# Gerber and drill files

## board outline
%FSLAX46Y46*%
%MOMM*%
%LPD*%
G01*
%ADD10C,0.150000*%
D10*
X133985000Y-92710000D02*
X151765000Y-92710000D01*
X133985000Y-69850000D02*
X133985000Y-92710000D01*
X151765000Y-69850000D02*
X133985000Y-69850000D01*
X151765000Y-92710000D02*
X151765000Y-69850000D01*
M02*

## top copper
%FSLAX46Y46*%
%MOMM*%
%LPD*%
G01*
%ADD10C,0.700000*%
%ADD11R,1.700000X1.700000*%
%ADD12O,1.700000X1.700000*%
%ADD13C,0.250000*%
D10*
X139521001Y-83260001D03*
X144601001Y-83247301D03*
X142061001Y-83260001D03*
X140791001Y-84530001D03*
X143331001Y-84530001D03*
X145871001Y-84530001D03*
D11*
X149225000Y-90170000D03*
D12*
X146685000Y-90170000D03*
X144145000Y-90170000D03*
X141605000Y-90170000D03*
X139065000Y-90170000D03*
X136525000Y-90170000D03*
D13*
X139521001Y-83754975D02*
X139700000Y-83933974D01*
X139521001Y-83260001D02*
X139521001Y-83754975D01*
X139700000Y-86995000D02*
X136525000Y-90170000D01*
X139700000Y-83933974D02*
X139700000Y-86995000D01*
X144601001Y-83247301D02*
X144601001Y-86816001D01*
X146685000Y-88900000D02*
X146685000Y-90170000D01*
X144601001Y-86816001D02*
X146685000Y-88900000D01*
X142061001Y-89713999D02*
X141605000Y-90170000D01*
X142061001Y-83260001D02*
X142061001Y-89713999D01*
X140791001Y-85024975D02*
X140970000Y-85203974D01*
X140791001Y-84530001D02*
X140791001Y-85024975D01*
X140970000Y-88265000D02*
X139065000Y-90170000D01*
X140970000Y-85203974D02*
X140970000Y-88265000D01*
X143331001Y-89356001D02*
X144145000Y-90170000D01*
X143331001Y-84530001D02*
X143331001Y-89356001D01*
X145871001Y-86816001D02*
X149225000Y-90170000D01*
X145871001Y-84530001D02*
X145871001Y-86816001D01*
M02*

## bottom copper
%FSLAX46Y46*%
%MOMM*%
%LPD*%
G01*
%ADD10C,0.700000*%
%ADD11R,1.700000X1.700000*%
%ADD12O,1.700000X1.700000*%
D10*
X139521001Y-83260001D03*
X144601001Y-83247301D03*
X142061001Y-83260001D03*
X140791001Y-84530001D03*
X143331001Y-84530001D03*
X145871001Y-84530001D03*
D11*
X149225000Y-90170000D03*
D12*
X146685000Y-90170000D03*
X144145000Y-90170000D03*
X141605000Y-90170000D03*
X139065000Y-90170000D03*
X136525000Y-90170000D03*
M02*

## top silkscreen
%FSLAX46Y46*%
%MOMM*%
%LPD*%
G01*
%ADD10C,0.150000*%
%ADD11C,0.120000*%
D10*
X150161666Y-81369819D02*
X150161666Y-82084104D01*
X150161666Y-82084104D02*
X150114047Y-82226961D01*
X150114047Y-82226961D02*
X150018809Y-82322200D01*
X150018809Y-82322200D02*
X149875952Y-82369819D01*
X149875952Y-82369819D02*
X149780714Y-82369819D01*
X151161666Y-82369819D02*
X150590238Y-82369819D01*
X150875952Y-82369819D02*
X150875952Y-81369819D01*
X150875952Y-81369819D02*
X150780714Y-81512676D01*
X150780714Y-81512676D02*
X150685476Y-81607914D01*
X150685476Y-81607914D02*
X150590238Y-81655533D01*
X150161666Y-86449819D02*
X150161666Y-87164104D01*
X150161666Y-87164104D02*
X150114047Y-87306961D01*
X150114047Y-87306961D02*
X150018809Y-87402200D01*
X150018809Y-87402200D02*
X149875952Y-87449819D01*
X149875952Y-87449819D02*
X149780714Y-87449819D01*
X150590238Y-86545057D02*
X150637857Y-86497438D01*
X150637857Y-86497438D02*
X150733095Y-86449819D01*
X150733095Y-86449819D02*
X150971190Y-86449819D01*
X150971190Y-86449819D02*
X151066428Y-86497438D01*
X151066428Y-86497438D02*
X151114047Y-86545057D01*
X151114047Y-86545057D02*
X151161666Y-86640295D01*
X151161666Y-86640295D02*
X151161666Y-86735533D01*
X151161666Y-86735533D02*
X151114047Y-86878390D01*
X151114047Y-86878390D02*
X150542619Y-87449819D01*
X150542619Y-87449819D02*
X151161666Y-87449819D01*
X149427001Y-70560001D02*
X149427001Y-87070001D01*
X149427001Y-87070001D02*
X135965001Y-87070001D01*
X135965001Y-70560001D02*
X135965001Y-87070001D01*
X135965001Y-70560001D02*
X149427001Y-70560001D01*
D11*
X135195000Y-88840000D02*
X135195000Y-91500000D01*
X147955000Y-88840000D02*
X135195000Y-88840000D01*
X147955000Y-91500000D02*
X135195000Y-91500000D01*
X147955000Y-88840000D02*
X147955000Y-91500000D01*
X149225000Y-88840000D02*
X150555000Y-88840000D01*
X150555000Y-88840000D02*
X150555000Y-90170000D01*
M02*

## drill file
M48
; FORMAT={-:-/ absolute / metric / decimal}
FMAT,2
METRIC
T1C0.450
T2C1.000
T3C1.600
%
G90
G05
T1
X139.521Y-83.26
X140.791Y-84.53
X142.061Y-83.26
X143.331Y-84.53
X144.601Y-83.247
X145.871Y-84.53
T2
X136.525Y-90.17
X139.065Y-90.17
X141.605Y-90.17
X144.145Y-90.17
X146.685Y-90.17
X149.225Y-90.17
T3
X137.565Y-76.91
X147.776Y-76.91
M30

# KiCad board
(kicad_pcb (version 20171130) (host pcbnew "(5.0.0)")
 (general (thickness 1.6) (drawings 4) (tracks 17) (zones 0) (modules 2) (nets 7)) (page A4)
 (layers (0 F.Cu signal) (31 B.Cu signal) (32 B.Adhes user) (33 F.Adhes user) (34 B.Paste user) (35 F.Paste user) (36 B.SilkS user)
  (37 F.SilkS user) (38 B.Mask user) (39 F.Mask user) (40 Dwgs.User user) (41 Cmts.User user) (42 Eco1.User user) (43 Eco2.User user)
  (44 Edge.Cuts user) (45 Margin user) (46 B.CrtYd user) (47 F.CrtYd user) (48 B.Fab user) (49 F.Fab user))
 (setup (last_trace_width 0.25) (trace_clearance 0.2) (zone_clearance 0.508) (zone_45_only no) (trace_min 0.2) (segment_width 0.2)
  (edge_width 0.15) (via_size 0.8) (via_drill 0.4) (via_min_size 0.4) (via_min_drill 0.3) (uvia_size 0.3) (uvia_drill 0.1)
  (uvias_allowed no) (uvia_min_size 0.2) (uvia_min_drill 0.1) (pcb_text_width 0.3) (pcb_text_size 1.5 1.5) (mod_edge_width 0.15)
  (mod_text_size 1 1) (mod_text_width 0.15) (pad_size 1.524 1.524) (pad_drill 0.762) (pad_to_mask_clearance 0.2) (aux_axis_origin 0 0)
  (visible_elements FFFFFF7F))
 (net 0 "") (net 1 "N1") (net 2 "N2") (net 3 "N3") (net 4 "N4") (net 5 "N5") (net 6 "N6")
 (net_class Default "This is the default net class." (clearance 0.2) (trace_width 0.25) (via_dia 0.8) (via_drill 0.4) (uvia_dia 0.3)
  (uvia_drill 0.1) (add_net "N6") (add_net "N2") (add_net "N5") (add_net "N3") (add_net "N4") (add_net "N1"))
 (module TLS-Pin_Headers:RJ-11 (layer F.Cu) (at 142.696001 83.260001)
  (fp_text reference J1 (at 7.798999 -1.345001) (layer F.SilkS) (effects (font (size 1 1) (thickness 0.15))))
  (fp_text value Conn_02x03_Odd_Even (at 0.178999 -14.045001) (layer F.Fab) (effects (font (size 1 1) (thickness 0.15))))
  (fp_line (start 6.731 -12.7) (end 6.731 3.81) (layer F.SilkS) (width 0.15))
  (fp_line (start 6.731 3.81) (end -6.731 3.81) (layer F.SilkS) (width 0.15))
  (fp_line (start -6.731 -12.7) (end -6.731 3.81) (layer F.SilkS) (width 0.15))
  (fp_line (start -6.731 -12.7) (end 6.731 -12.7) (layer F.SilkS) (width 0.15))
  (pad "" np_thru_hole circle (at 5.08 -6.35) (size 1.6 1.6) (drill 1.6) (layers *.Cu *.Mask))
  (pad "" np_thru_hole circle (at -5.1308 -6.35) (size 1.6 1.6) (drill 1.6) (layers *.Cu *.Mask))
  (pad 6 thru_hole circle (at -3.175 0) (size 0.7 0.7) (drill 0.45) (layers *.Cu *.Mask) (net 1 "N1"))
  (pad 2 thru_hole circle (at 1.905 -0.0127) (size 0.7 0.7) (drill 0.45) (layers *.Cu *.Mask) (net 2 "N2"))
  (pad 4 thru_hole circle (at -0.635 0) (size 0.7 0.7) (drill 0.45) (layers *.Cu *.Mask) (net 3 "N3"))
  (pad 5 thru_hole circle (at -1.905 1.27) (size 0.7 0.7) (drill 0.45) (layers *.Cu *.Mask) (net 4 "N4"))
  (pad 3 thru_hole circle (at 0.635 1.27) (size 0.7 0.7) (drill 0.45) (layers *.Cu *.Mask) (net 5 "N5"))
  (pad 1 thru_hole circle (at 3.175 1.27) (size 0.7 0.7) (drill 0.45) (layers *.Cu *.Mask) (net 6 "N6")))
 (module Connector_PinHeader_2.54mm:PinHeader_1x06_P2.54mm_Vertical (layer F.Cu) (at 149.225 90.17 270)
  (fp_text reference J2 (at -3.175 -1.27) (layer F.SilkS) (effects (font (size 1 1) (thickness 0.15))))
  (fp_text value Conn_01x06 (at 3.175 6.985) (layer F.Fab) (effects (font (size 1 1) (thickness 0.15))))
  (fp_line (start -1.33 14.03) (end 1.33 14.03) (layer F.SilkS) (width 0.12))
  (fp_line (start -1.33 1.27) (end -1.33 14.03) (layer F.SilkS) (width 0.12))
  (fp_line (start 1.33 1.27) (end 1.33 14.03) (layer F.SilkS) (width 0.12))
  (fp_line (start -1.33 1.27) (end 1.33 1.27) (layer F.SilkS) (width 0.12))
  (fp_line (start -1.33 0) (end -1.33 -1.33) (layer F.SilkS) (width 0.12))
  (fp_line (start -1.33 -1.33) (end 0 -1.33) (layer F.SilkS) (width 0.12))
  (pad 1 thru_hole rect (at 0 0 270) (size 1.7 1.7) (drill 1) (layers *.Cu *.Mask) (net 6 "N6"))
  (pad 2 thru_hole oval (at 0 2.54 270) (size 1.7 1.7) (drill 1) (layers *.Cu *.Mask) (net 2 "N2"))
  (pad 3 thru_hole oval (at 0 5.08 270) (size 1.7 1.7) (drill 1) (layers *.Cu *.Mask) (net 5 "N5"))
  (pad 4 thru_hole oval (at 0 7.62 270) (size 1.7 1.7) (drill 1) (layers *.Cu *.Mask) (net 3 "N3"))
  (pad 5 thru_hole oval (at 0 10.16 270) (size 1.7 1.7) (drill 1) (layers *.Cu *.Mask) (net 4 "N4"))
  (pad 6 thru_hole oval (at 0 12.7 270) (size 1.7 1.7) (drill 1) (layers *.Cu *.Mask) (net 1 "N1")))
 (gr_line (start 133.985 92.71) (end 151.765 92.71) (layer Edge.Cuts) (width 0.15))
 (gr_line (start 133.985 69.85) (end 133.985 92.71) (layer Edge.Cuts) (width 0.15))
 (gr_line (start 151.765 69.85) (end 133.985 69.85) (layer Edge.Cuts) (width 0.15))
 (gr_line (start 151.765 92.71) (end 151.765 69.85) (layer Edge.Cuts) (width 0.15))
 (segment (start 139.521001 83.754975) (end 139.7 83.933974) (width 0.25) (layer F.Cu) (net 1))
 (segment (start 139.521001 83.260001) (end 139.521001 83.754975) (width 0.25) (layer F.Cu) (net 1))
 (segment (start 139.7 86.995) (end 136.525 90.17) (width 0.25) (layer F.Cu) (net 1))
 (segment (start 139.7 83.933974) (end 139.7 86.995) (width 0.25) (layer F.Cu) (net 1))
 (segment (start 144.601001 83.247301) (end 144.601001 86.816001) (width 0.25) (layer F.Cu) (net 2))
 (segment (start 146.685 88.9) (end 146.685 90.17) (width 0.25) (layer F.Cu) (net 2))
 (segment (start 144.601001 86.816001) (end 146.685 88.9) (width 0.25) (layer F.Cu) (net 2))
 (segment (start 142.061001 89.713999) (end 141.605 90.17) (width 0.25) (layer F.Cu) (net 3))
 (segment (start 142.061001 83.260001) (end 142.061001 89.713999) (width 0.25) (layer F.Cu) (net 3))
 (segment (start 140.791001 85.024975) (end 140.97 85.203974) (width 0.25) (layer F.Cu) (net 4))
 (segment (start 140.791001 84.530001) (end 140.791001 85.024975) (width 0.25) (layer F.Cu) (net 4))
 (segment (start 140.97 88.265) (end 139.065 90.17) (width 0.25) (layer F.Cu) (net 4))
 (segment (start 140.97 85.203974) (end 140.97 88.265) (width 0.25) (layer F.Cu) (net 4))
 (segment (start 143.331001 89.356001) (end 144.145 90.17) (width 0.25) (layer F.Cu) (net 5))
 (segment (start 143.331001 84.530001) (end 143.331001 89.356001) (width 0.25) (layer F.Cu) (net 5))
 (segment (start 145.871001 86.816001) (end 149.225 90.17) (width 0.25) (layer F.Cu) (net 6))
 (segment (start 145.871001 84.530001) (end 145.871001 86.816001) (width 0.25) (layer F.Cu) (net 6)))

